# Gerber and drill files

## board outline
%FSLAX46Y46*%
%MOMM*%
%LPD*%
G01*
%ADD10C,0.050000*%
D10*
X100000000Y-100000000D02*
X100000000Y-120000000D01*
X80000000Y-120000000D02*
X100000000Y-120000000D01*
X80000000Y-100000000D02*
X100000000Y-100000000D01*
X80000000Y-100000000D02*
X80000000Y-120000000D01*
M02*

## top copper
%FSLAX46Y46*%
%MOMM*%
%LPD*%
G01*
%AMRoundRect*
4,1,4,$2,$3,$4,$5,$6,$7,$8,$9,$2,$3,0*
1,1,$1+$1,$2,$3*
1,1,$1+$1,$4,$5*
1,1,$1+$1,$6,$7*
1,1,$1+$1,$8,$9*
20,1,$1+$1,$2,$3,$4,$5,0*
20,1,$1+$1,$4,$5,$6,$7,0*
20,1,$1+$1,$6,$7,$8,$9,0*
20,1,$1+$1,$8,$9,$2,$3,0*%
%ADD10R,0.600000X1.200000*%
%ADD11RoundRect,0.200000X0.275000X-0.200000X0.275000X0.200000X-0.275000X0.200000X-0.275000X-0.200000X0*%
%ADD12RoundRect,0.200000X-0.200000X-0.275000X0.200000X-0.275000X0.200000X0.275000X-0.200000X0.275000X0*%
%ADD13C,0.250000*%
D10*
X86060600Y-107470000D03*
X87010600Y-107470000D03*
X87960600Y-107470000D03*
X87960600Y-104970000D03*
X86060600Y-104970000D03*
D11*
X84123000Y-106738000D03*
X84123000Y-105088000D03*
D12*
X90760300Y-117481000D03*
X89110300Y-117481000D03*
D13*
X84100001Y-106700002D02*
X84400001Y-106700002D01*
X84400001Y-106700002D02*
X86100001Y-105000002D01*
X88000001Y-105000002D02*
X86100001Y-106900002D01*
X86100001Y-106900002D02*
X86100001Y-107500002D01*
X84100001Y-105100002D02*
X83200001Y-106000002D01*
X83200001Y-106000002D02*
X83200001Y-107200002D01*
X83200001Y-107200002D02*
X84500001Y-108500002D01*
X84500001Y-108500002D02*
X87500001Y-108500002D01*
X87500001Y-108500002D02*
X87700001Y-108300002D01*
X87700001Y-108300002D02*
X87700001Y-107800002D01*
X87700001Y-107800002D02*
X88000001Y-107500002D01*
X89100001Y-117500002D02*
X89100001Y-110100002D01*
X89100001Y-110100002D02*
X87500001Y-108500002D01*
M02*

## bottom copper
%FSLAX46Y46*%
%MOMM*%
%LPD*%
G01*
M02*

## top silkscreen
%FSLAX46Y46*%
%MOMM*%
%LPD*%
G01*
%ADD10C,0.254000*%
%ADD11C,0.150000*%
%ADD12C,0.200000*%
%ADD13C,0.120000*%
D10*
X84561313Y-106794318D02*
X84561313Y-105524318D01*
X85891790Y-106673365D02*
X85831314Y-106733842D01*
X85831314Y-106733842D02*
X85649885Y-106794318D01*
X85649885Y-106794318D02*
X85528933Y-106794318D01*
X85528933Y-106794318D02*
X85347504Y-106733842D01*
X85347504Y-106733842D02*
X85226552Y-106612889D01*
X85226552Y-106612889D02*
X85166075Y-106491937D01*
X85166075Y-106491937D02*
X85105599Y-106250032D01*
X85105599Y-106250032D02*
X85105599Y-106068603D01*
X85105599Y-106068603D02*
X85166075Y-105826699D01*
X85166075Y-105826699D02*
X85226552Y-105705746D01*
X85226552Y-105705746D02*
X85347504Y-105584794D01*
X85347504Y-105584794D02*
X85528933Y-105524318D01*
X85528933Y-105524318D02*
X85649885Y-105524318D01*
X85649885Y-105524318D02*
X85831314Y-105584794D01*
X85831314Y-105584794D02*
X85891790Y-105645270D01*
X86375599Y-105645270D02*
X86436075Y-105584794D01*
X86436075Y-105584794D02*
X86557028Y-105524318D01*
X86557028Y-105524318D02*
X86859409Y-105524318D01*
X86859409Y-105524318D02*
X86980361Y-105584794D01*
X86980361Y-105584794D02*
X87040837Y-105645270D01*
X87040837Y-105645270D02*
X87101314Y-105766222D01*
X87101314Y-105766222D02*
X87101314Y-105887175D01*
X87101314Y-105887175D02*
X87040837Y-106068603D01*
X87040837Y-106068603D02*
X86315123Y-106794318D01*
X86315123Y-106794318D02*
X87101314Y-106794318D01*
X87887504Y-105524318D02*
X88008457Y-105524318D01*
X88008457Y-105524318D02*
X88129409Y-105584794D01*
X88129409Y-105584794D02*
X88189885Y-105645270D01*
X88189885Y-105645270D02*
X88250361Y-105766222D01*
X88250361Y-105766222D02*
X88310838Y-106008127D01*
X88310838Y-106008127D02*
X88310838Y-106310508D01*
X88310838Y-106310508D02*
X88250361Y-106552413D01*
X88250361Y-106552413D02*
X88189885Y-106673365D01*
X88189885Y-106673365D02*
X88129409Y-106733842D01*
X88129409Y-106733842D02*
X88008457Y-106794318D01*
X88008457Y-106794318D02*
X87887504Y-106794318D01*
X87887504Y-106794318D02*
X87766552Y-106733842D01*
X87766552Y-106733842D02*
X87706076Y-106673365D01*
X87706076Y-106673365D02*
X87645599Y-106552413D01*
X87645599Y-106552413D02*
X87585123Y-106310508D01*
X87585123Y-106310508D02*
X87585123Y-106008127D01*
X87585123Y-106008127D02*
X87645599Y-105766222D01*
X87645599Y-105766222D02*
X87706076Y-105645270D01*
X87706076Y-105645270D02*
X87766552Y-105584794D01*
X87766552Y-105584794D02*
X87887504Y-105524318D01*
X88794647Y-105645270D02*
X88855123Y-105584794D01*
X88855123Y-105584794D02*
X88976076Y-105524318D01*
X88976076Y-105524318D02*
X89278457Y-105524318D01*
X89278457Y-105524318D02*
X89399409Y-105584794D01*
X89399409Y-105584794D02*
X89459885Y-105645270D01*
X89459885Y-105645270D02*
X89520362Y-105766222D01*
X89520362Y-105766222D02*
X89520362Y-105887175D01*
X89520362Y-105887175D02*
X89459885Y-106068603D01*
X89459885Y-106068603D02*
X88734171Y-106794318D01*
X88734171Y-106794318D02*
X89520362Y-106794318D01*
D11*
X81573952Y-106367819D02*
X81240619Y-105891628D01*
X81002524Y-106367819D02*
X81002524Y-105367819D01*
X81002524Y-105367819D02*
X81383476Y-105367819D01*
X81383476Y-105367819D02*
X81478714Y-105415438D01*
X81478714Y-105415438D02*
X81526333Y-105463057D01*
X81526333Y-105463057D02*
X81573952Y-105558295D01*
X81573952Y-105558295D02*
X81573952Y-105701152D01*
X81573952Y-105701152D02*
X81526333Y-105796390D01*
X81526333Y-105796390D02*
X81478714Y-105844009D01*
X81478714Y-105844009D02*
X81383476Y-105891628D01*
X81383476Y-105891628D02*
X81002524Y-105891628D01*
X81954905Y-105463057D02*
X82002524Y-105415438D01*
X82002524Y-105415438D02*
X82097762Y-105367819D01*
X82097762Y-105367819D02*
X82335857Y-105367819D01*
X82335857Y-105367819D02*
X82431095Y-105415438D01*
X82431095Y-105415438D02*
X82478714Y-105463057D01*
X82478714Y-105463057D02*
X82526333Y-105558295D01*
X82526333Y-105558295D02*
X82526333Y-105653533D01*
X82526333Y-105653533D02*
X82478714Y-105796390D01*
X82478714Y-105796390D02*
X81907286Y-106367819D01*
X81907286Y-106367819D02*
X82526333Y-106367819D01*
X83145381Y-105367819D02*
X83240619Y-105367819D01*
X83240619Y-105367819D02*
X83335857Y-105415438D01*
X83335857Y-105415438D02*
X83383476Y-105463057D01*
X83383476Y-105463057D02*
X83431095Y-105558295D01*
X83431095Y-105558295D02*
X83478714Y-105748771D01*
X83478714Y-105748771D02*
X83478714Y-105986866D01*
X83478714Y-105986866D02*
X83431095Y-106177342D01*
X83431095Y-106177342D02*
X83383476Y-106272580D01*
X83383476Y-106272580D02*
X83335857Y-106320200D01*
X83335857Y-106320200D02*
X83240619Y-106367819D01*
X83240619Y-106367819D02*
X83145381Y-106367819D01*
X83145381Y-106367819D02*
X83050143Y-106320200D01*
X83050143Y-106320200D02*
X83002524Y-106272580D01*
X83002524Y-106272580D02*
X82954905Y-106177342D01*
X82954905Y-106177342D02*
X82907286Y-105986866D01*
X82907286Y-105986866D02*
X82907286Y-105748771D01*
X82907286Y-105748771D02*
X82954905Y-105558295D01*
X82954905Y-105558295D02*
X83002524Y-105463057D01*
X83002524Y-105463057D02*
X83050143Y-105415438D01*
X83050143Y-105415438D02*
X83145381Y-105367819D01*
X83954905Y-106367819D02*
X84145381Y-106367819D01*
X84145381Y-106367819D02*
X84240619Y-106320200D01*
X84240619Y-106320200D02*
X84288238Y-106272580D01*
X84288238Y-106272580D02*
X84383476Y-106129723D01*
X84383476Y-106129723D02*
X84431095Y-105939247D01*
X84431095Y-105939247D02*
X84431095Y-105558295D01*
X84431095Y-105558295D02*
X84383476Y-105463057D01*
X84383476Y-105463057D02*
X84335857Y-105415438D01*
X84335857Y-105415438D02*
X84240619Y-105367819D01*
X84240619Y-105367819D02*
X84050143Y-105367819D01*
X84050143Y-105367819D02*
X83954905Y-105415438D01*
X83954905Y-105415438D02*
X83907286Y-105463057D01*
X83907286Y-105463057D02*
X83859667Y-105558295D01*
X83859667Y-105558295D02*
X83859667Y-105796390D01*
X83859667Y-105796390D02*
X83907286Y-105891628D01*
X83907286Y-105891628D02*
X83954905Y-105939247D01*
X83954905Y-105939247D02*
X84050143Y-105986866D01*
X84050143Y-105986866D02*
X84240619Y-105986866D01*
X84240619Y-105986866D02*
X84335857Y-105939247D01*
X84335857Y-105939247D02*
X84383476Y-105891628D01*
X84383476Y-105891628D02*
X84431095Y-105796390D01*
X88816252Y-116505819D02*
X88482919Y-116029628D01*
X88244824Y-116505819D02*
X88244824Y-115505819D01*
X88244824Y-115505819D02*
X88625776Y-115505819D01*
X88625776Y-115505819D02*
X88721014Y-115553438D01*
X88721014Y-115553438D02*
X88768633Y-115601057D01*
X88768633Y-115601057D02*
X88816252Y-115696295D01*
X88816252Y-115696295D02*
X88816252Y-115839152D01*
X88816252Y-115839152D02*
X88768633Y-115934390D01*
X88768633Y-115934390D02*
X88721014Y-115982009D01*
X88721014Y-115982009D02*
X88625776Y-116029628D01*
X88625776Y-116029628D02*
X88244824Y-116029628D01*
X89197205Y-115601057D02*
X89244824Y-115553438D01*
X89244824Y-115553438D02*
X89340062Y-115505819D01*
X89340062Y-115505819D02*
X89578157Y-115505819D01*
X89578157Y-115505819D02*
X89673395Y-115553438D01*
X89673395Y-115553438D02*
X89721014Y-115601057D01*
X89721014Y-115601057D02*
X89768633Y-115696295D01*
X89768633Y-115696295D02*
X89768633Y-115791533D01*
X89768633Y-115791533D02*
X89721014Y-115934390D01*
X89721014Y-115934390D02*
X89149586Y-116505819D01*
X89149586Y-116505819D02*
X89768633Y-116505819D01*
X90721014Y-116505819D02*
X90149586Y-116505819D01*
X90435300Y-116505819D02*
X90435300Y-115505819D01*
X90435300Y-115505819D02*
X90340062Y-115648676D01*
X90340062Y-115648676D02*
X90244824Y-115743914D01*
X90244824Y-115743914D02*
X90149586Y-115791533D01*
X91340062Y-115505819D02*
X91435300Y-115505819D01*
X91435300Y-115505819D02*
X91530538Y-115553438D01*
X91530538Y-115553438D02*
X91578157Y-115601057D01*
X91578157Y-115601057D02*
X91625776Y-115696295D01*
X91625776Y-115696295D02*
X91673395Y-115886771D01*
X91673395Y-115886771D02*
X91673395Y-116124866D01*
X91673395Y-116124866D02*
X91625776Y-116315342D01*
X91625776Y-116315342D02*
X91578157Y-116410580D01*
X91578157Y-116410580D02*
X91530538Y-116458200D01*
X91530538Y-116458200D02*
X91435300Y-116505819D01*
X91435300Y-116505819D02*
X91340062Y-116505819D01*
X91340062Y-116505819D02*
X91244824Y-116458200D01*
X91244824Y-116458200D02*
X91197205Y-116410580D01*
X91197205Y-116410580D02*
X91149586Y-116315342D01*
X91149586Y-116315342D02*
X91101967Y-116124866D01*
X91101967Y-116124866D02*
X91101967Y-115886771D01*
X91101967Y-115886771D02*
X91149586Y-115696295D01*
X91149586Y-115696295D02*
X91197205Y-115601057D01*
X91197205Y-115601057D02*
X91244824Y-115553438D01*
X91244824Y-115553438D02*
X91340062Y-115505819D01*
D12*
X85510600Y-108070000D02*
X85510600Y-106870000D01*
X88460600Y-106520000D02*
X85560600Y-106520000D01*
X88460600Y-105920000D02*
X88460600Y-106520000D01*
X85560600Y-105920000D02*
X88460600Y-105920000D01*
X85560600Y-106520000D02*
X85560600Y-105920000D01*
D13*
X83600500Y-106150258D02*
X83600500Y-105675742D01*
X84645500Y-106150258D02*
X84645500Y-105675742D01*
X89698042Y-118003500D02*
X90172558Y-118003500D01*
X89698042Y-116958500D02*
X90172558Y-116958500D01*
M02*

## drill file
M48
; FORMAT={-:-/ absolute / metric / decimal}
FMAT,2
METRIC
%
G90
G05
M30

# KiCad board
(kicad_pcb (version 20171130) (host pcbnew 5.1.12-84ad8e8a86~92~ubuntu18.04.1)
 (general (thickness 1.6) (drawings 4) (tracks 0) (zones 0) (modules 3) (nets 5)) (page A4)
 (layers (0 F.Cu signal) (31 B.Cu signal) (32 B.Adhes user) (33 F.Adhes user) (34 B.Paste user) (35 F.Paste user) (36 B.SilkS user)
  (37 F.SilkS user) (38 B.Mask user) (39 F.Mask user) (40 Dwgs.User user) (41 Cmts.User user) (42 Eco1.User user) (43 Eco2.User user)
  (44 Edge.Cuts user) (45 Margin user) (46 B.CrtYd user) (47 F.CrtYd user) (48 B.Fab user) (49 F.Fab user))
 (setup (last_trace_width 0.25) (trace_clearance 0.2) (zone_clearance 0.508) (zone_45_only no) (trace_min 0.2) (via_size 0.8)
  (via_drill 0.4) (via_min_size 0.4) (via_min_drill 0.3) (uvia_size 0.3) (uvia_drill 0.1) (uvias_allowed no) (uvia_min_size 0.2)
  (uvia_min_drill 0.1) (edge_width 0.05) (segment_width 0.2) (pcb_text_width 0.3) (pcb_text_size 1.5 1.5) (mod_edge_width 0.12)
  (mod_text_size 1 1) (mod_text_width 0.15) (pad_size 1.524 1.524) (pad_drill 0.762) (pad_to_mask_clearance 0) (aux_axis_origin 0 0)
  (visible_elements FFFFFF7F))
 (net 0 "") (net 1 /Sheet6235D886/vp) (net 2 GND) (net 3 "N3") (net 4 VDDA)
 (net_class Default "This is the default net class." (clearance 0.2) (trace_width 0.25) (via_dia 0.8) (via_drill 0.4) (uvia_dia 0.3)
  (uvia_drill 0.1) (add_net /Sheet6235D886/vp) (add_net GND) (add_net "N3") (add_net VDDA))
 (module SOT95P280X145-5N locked (layer F.Cu) (at 87.010600 106.220000 90.000000)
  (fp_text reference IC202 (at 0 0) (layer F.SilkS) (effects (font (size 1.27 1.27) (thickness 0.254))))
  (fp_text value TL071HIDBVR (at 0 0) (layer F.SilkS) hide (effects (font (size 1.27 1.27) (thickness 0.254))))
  (fp_line (start -1.85 -1.5) (end -0.65 -1.5) (layer F.SilkS) (width 0.2))
  (fp_line (start -0.3 1.45) (end -0.3 -1.45) (layer F.SilkS) (width 0.2))
  (fp_line (start 0.3 1.45) (end -0.3 1.45) (layer F.SilkS) (width 0.2))
  (fp_line (start 0.3 -1.45) (end 0.3 1.45) (layer F.SilkS) (width 0.2))
  (fp_line (start -0.3 -1.45) (end 0.3 -1.45) (layer F.SilkS) (width 0.2))
  (pad 1 smd rect (at -1.25 -0.95 180.000000) (size 0.6 1.2) (layers F.Cu F.Mask F.Paste) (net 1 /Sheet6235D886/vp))
  (pad 2 smd rect (at -1.25 0 180.000000) (size 0.6 1.2) (layers F.Cu F.Mask F.Paste) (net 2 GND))
  (pad 3 smd rect (at -1.25 0.95 180.000000) (size 0.6 1.2) (layers F.Cu F.Mask F.Paste) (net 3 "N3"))
  (pad 4 smd rect (at 1.25 0.95 180.000000) (size 0.6 1.2) (layers F.Cu F.Mask F.Paste) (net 1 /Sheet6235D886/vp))
  (pad 5 smd rect (at 1.25 -0.95 180.000000) (size 0.6 1.2) (layers F.Cu F.Mask F.Paste) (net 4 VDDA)))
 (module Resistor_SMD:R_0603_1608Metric (layer F.Cu) (at 84.123000 105.913000 90.000000)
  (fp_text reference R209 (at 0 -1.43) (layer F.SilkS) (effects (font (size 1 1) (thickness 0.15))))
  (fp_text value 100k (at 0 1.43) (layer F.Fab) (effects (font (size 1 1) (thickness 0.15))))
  (fp_line (start -0.237258 -0.5225) (end 0.237258 -0.5225) (layer F.SilkS) (width 0.12))
  (fp_line (start -0.237258 0.5225) (end 0.237258 0.5225) (layer F.SilkS) (width 0.12))
  (pad 1 smd roundrect (at -0.825 0 90.000000) (size 0.8 0.95) (layers F.Cu F.Mask F.Paste) (roundrect_rratio 0.25) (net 4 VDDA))
  (pad 2 smd roundrect (at 0.825 0 90.000000) (size 0.8 0.95) (layers F.Cu F.Mask F.Paste) (roundrect_rratio 0.25) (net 3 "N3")))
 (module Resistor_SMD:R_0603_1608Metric (layer F.Cu) (at 89.935300 117.481000)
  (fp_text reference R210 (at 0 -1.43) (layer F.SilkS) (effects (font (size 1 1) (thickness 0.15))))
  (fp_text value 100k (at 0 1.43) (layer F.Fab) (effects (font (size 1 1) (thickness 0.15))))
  (fp_line (start -0.237258 0.5225) (end 0.237258 0.5225) (layer F.SilkS) (width 0.12))
  (fp_line (start -0.237258 -0.5225) (end 0.237258 -0.5225) (layer F.SilkS) (width 0.12))
  (pad 2 smd roundrect (at 0.825 0) (size 0.8 0.95) (layers F.Cu F.Mask F.Paste) (roundrect_rratio 0.25) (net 2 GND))
  (pad 1 smd roundrect (at -0.825 0) (size 0.8 0.95) (layers F.Cu F.Mask F.Paste) (roundrect_rratio 0.25) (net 3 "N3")))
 (gr_line (start 100 100) (end 100 120) (layer Edge.Cuts) (width 0.05))
 (gr_line (start 80 120) (end 100 120) (layer Edge.Cuts) (width 0.05))
 (gr_line (start 80 100) (end 100 100) (layer Edge.Cuts) (width 0.05))
 (gr_line (start 80 100) (end 80 120) (layer Edge.Cuts) (width 0.05))
 (segment (start 84.100001 106.700002) (end 84.400001 106.700002) (width 0.250000) (layer F.Cu) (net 4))
 (segment (start 84.400001 106.700002) (end 86.100001 105.000002) (width 0.250000) (layer F.Cu) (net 4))
 (segment (start 88.000001 105.000002) (end 86.100001 106.900002) (width 0.250000) (layer F.Cu) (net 1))
 (segment (start 86.100001 106.900002) (end 86.100001 107.500002) (width 0.250000) (layer F.Cu) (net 1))
 (segment (start 84.100001 105.100002) (end 83.200001 106.000002) (width 0.250000) (layer F.Cu) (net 3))
 (segment (start 83.200001 106.000002) (end 83.200001 107.200002) (width 0.250000) (layer F.Cu) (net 3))
 (segment (start 83.200001 107.200002) (end 84.500001 108.500002) (width 0.250000) (layer F.Cu) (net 3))
 (segment (start 84.500001 108.500002) (end 87.500001 108.500002) (width 0.250000) (layer F.Cu) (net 3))
 (segment (start 87.500001 108.500002) (end 87.700001 108.300002) (width 0.250000) (layer F.Cu) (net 3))
 (segment (start 87.700001 108.300002) (end 87.700001 107.800002) (width 0.250000) (layer F.Cu) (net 3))
 (segment (start 87.700001 107.800002) (end 88.000001 107.500002) (width 0.250000) (layer F.Cu) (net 3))
 (segment (start 89.100001 117.500002) (end 89.100001 110.100002) (width 0.250000) (layer F.Cu) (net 3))
 (segment (start 89.100001 110.100002) (end 87.500001 108.500002) (width 0.250000) (layer F.Cu) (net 3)))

